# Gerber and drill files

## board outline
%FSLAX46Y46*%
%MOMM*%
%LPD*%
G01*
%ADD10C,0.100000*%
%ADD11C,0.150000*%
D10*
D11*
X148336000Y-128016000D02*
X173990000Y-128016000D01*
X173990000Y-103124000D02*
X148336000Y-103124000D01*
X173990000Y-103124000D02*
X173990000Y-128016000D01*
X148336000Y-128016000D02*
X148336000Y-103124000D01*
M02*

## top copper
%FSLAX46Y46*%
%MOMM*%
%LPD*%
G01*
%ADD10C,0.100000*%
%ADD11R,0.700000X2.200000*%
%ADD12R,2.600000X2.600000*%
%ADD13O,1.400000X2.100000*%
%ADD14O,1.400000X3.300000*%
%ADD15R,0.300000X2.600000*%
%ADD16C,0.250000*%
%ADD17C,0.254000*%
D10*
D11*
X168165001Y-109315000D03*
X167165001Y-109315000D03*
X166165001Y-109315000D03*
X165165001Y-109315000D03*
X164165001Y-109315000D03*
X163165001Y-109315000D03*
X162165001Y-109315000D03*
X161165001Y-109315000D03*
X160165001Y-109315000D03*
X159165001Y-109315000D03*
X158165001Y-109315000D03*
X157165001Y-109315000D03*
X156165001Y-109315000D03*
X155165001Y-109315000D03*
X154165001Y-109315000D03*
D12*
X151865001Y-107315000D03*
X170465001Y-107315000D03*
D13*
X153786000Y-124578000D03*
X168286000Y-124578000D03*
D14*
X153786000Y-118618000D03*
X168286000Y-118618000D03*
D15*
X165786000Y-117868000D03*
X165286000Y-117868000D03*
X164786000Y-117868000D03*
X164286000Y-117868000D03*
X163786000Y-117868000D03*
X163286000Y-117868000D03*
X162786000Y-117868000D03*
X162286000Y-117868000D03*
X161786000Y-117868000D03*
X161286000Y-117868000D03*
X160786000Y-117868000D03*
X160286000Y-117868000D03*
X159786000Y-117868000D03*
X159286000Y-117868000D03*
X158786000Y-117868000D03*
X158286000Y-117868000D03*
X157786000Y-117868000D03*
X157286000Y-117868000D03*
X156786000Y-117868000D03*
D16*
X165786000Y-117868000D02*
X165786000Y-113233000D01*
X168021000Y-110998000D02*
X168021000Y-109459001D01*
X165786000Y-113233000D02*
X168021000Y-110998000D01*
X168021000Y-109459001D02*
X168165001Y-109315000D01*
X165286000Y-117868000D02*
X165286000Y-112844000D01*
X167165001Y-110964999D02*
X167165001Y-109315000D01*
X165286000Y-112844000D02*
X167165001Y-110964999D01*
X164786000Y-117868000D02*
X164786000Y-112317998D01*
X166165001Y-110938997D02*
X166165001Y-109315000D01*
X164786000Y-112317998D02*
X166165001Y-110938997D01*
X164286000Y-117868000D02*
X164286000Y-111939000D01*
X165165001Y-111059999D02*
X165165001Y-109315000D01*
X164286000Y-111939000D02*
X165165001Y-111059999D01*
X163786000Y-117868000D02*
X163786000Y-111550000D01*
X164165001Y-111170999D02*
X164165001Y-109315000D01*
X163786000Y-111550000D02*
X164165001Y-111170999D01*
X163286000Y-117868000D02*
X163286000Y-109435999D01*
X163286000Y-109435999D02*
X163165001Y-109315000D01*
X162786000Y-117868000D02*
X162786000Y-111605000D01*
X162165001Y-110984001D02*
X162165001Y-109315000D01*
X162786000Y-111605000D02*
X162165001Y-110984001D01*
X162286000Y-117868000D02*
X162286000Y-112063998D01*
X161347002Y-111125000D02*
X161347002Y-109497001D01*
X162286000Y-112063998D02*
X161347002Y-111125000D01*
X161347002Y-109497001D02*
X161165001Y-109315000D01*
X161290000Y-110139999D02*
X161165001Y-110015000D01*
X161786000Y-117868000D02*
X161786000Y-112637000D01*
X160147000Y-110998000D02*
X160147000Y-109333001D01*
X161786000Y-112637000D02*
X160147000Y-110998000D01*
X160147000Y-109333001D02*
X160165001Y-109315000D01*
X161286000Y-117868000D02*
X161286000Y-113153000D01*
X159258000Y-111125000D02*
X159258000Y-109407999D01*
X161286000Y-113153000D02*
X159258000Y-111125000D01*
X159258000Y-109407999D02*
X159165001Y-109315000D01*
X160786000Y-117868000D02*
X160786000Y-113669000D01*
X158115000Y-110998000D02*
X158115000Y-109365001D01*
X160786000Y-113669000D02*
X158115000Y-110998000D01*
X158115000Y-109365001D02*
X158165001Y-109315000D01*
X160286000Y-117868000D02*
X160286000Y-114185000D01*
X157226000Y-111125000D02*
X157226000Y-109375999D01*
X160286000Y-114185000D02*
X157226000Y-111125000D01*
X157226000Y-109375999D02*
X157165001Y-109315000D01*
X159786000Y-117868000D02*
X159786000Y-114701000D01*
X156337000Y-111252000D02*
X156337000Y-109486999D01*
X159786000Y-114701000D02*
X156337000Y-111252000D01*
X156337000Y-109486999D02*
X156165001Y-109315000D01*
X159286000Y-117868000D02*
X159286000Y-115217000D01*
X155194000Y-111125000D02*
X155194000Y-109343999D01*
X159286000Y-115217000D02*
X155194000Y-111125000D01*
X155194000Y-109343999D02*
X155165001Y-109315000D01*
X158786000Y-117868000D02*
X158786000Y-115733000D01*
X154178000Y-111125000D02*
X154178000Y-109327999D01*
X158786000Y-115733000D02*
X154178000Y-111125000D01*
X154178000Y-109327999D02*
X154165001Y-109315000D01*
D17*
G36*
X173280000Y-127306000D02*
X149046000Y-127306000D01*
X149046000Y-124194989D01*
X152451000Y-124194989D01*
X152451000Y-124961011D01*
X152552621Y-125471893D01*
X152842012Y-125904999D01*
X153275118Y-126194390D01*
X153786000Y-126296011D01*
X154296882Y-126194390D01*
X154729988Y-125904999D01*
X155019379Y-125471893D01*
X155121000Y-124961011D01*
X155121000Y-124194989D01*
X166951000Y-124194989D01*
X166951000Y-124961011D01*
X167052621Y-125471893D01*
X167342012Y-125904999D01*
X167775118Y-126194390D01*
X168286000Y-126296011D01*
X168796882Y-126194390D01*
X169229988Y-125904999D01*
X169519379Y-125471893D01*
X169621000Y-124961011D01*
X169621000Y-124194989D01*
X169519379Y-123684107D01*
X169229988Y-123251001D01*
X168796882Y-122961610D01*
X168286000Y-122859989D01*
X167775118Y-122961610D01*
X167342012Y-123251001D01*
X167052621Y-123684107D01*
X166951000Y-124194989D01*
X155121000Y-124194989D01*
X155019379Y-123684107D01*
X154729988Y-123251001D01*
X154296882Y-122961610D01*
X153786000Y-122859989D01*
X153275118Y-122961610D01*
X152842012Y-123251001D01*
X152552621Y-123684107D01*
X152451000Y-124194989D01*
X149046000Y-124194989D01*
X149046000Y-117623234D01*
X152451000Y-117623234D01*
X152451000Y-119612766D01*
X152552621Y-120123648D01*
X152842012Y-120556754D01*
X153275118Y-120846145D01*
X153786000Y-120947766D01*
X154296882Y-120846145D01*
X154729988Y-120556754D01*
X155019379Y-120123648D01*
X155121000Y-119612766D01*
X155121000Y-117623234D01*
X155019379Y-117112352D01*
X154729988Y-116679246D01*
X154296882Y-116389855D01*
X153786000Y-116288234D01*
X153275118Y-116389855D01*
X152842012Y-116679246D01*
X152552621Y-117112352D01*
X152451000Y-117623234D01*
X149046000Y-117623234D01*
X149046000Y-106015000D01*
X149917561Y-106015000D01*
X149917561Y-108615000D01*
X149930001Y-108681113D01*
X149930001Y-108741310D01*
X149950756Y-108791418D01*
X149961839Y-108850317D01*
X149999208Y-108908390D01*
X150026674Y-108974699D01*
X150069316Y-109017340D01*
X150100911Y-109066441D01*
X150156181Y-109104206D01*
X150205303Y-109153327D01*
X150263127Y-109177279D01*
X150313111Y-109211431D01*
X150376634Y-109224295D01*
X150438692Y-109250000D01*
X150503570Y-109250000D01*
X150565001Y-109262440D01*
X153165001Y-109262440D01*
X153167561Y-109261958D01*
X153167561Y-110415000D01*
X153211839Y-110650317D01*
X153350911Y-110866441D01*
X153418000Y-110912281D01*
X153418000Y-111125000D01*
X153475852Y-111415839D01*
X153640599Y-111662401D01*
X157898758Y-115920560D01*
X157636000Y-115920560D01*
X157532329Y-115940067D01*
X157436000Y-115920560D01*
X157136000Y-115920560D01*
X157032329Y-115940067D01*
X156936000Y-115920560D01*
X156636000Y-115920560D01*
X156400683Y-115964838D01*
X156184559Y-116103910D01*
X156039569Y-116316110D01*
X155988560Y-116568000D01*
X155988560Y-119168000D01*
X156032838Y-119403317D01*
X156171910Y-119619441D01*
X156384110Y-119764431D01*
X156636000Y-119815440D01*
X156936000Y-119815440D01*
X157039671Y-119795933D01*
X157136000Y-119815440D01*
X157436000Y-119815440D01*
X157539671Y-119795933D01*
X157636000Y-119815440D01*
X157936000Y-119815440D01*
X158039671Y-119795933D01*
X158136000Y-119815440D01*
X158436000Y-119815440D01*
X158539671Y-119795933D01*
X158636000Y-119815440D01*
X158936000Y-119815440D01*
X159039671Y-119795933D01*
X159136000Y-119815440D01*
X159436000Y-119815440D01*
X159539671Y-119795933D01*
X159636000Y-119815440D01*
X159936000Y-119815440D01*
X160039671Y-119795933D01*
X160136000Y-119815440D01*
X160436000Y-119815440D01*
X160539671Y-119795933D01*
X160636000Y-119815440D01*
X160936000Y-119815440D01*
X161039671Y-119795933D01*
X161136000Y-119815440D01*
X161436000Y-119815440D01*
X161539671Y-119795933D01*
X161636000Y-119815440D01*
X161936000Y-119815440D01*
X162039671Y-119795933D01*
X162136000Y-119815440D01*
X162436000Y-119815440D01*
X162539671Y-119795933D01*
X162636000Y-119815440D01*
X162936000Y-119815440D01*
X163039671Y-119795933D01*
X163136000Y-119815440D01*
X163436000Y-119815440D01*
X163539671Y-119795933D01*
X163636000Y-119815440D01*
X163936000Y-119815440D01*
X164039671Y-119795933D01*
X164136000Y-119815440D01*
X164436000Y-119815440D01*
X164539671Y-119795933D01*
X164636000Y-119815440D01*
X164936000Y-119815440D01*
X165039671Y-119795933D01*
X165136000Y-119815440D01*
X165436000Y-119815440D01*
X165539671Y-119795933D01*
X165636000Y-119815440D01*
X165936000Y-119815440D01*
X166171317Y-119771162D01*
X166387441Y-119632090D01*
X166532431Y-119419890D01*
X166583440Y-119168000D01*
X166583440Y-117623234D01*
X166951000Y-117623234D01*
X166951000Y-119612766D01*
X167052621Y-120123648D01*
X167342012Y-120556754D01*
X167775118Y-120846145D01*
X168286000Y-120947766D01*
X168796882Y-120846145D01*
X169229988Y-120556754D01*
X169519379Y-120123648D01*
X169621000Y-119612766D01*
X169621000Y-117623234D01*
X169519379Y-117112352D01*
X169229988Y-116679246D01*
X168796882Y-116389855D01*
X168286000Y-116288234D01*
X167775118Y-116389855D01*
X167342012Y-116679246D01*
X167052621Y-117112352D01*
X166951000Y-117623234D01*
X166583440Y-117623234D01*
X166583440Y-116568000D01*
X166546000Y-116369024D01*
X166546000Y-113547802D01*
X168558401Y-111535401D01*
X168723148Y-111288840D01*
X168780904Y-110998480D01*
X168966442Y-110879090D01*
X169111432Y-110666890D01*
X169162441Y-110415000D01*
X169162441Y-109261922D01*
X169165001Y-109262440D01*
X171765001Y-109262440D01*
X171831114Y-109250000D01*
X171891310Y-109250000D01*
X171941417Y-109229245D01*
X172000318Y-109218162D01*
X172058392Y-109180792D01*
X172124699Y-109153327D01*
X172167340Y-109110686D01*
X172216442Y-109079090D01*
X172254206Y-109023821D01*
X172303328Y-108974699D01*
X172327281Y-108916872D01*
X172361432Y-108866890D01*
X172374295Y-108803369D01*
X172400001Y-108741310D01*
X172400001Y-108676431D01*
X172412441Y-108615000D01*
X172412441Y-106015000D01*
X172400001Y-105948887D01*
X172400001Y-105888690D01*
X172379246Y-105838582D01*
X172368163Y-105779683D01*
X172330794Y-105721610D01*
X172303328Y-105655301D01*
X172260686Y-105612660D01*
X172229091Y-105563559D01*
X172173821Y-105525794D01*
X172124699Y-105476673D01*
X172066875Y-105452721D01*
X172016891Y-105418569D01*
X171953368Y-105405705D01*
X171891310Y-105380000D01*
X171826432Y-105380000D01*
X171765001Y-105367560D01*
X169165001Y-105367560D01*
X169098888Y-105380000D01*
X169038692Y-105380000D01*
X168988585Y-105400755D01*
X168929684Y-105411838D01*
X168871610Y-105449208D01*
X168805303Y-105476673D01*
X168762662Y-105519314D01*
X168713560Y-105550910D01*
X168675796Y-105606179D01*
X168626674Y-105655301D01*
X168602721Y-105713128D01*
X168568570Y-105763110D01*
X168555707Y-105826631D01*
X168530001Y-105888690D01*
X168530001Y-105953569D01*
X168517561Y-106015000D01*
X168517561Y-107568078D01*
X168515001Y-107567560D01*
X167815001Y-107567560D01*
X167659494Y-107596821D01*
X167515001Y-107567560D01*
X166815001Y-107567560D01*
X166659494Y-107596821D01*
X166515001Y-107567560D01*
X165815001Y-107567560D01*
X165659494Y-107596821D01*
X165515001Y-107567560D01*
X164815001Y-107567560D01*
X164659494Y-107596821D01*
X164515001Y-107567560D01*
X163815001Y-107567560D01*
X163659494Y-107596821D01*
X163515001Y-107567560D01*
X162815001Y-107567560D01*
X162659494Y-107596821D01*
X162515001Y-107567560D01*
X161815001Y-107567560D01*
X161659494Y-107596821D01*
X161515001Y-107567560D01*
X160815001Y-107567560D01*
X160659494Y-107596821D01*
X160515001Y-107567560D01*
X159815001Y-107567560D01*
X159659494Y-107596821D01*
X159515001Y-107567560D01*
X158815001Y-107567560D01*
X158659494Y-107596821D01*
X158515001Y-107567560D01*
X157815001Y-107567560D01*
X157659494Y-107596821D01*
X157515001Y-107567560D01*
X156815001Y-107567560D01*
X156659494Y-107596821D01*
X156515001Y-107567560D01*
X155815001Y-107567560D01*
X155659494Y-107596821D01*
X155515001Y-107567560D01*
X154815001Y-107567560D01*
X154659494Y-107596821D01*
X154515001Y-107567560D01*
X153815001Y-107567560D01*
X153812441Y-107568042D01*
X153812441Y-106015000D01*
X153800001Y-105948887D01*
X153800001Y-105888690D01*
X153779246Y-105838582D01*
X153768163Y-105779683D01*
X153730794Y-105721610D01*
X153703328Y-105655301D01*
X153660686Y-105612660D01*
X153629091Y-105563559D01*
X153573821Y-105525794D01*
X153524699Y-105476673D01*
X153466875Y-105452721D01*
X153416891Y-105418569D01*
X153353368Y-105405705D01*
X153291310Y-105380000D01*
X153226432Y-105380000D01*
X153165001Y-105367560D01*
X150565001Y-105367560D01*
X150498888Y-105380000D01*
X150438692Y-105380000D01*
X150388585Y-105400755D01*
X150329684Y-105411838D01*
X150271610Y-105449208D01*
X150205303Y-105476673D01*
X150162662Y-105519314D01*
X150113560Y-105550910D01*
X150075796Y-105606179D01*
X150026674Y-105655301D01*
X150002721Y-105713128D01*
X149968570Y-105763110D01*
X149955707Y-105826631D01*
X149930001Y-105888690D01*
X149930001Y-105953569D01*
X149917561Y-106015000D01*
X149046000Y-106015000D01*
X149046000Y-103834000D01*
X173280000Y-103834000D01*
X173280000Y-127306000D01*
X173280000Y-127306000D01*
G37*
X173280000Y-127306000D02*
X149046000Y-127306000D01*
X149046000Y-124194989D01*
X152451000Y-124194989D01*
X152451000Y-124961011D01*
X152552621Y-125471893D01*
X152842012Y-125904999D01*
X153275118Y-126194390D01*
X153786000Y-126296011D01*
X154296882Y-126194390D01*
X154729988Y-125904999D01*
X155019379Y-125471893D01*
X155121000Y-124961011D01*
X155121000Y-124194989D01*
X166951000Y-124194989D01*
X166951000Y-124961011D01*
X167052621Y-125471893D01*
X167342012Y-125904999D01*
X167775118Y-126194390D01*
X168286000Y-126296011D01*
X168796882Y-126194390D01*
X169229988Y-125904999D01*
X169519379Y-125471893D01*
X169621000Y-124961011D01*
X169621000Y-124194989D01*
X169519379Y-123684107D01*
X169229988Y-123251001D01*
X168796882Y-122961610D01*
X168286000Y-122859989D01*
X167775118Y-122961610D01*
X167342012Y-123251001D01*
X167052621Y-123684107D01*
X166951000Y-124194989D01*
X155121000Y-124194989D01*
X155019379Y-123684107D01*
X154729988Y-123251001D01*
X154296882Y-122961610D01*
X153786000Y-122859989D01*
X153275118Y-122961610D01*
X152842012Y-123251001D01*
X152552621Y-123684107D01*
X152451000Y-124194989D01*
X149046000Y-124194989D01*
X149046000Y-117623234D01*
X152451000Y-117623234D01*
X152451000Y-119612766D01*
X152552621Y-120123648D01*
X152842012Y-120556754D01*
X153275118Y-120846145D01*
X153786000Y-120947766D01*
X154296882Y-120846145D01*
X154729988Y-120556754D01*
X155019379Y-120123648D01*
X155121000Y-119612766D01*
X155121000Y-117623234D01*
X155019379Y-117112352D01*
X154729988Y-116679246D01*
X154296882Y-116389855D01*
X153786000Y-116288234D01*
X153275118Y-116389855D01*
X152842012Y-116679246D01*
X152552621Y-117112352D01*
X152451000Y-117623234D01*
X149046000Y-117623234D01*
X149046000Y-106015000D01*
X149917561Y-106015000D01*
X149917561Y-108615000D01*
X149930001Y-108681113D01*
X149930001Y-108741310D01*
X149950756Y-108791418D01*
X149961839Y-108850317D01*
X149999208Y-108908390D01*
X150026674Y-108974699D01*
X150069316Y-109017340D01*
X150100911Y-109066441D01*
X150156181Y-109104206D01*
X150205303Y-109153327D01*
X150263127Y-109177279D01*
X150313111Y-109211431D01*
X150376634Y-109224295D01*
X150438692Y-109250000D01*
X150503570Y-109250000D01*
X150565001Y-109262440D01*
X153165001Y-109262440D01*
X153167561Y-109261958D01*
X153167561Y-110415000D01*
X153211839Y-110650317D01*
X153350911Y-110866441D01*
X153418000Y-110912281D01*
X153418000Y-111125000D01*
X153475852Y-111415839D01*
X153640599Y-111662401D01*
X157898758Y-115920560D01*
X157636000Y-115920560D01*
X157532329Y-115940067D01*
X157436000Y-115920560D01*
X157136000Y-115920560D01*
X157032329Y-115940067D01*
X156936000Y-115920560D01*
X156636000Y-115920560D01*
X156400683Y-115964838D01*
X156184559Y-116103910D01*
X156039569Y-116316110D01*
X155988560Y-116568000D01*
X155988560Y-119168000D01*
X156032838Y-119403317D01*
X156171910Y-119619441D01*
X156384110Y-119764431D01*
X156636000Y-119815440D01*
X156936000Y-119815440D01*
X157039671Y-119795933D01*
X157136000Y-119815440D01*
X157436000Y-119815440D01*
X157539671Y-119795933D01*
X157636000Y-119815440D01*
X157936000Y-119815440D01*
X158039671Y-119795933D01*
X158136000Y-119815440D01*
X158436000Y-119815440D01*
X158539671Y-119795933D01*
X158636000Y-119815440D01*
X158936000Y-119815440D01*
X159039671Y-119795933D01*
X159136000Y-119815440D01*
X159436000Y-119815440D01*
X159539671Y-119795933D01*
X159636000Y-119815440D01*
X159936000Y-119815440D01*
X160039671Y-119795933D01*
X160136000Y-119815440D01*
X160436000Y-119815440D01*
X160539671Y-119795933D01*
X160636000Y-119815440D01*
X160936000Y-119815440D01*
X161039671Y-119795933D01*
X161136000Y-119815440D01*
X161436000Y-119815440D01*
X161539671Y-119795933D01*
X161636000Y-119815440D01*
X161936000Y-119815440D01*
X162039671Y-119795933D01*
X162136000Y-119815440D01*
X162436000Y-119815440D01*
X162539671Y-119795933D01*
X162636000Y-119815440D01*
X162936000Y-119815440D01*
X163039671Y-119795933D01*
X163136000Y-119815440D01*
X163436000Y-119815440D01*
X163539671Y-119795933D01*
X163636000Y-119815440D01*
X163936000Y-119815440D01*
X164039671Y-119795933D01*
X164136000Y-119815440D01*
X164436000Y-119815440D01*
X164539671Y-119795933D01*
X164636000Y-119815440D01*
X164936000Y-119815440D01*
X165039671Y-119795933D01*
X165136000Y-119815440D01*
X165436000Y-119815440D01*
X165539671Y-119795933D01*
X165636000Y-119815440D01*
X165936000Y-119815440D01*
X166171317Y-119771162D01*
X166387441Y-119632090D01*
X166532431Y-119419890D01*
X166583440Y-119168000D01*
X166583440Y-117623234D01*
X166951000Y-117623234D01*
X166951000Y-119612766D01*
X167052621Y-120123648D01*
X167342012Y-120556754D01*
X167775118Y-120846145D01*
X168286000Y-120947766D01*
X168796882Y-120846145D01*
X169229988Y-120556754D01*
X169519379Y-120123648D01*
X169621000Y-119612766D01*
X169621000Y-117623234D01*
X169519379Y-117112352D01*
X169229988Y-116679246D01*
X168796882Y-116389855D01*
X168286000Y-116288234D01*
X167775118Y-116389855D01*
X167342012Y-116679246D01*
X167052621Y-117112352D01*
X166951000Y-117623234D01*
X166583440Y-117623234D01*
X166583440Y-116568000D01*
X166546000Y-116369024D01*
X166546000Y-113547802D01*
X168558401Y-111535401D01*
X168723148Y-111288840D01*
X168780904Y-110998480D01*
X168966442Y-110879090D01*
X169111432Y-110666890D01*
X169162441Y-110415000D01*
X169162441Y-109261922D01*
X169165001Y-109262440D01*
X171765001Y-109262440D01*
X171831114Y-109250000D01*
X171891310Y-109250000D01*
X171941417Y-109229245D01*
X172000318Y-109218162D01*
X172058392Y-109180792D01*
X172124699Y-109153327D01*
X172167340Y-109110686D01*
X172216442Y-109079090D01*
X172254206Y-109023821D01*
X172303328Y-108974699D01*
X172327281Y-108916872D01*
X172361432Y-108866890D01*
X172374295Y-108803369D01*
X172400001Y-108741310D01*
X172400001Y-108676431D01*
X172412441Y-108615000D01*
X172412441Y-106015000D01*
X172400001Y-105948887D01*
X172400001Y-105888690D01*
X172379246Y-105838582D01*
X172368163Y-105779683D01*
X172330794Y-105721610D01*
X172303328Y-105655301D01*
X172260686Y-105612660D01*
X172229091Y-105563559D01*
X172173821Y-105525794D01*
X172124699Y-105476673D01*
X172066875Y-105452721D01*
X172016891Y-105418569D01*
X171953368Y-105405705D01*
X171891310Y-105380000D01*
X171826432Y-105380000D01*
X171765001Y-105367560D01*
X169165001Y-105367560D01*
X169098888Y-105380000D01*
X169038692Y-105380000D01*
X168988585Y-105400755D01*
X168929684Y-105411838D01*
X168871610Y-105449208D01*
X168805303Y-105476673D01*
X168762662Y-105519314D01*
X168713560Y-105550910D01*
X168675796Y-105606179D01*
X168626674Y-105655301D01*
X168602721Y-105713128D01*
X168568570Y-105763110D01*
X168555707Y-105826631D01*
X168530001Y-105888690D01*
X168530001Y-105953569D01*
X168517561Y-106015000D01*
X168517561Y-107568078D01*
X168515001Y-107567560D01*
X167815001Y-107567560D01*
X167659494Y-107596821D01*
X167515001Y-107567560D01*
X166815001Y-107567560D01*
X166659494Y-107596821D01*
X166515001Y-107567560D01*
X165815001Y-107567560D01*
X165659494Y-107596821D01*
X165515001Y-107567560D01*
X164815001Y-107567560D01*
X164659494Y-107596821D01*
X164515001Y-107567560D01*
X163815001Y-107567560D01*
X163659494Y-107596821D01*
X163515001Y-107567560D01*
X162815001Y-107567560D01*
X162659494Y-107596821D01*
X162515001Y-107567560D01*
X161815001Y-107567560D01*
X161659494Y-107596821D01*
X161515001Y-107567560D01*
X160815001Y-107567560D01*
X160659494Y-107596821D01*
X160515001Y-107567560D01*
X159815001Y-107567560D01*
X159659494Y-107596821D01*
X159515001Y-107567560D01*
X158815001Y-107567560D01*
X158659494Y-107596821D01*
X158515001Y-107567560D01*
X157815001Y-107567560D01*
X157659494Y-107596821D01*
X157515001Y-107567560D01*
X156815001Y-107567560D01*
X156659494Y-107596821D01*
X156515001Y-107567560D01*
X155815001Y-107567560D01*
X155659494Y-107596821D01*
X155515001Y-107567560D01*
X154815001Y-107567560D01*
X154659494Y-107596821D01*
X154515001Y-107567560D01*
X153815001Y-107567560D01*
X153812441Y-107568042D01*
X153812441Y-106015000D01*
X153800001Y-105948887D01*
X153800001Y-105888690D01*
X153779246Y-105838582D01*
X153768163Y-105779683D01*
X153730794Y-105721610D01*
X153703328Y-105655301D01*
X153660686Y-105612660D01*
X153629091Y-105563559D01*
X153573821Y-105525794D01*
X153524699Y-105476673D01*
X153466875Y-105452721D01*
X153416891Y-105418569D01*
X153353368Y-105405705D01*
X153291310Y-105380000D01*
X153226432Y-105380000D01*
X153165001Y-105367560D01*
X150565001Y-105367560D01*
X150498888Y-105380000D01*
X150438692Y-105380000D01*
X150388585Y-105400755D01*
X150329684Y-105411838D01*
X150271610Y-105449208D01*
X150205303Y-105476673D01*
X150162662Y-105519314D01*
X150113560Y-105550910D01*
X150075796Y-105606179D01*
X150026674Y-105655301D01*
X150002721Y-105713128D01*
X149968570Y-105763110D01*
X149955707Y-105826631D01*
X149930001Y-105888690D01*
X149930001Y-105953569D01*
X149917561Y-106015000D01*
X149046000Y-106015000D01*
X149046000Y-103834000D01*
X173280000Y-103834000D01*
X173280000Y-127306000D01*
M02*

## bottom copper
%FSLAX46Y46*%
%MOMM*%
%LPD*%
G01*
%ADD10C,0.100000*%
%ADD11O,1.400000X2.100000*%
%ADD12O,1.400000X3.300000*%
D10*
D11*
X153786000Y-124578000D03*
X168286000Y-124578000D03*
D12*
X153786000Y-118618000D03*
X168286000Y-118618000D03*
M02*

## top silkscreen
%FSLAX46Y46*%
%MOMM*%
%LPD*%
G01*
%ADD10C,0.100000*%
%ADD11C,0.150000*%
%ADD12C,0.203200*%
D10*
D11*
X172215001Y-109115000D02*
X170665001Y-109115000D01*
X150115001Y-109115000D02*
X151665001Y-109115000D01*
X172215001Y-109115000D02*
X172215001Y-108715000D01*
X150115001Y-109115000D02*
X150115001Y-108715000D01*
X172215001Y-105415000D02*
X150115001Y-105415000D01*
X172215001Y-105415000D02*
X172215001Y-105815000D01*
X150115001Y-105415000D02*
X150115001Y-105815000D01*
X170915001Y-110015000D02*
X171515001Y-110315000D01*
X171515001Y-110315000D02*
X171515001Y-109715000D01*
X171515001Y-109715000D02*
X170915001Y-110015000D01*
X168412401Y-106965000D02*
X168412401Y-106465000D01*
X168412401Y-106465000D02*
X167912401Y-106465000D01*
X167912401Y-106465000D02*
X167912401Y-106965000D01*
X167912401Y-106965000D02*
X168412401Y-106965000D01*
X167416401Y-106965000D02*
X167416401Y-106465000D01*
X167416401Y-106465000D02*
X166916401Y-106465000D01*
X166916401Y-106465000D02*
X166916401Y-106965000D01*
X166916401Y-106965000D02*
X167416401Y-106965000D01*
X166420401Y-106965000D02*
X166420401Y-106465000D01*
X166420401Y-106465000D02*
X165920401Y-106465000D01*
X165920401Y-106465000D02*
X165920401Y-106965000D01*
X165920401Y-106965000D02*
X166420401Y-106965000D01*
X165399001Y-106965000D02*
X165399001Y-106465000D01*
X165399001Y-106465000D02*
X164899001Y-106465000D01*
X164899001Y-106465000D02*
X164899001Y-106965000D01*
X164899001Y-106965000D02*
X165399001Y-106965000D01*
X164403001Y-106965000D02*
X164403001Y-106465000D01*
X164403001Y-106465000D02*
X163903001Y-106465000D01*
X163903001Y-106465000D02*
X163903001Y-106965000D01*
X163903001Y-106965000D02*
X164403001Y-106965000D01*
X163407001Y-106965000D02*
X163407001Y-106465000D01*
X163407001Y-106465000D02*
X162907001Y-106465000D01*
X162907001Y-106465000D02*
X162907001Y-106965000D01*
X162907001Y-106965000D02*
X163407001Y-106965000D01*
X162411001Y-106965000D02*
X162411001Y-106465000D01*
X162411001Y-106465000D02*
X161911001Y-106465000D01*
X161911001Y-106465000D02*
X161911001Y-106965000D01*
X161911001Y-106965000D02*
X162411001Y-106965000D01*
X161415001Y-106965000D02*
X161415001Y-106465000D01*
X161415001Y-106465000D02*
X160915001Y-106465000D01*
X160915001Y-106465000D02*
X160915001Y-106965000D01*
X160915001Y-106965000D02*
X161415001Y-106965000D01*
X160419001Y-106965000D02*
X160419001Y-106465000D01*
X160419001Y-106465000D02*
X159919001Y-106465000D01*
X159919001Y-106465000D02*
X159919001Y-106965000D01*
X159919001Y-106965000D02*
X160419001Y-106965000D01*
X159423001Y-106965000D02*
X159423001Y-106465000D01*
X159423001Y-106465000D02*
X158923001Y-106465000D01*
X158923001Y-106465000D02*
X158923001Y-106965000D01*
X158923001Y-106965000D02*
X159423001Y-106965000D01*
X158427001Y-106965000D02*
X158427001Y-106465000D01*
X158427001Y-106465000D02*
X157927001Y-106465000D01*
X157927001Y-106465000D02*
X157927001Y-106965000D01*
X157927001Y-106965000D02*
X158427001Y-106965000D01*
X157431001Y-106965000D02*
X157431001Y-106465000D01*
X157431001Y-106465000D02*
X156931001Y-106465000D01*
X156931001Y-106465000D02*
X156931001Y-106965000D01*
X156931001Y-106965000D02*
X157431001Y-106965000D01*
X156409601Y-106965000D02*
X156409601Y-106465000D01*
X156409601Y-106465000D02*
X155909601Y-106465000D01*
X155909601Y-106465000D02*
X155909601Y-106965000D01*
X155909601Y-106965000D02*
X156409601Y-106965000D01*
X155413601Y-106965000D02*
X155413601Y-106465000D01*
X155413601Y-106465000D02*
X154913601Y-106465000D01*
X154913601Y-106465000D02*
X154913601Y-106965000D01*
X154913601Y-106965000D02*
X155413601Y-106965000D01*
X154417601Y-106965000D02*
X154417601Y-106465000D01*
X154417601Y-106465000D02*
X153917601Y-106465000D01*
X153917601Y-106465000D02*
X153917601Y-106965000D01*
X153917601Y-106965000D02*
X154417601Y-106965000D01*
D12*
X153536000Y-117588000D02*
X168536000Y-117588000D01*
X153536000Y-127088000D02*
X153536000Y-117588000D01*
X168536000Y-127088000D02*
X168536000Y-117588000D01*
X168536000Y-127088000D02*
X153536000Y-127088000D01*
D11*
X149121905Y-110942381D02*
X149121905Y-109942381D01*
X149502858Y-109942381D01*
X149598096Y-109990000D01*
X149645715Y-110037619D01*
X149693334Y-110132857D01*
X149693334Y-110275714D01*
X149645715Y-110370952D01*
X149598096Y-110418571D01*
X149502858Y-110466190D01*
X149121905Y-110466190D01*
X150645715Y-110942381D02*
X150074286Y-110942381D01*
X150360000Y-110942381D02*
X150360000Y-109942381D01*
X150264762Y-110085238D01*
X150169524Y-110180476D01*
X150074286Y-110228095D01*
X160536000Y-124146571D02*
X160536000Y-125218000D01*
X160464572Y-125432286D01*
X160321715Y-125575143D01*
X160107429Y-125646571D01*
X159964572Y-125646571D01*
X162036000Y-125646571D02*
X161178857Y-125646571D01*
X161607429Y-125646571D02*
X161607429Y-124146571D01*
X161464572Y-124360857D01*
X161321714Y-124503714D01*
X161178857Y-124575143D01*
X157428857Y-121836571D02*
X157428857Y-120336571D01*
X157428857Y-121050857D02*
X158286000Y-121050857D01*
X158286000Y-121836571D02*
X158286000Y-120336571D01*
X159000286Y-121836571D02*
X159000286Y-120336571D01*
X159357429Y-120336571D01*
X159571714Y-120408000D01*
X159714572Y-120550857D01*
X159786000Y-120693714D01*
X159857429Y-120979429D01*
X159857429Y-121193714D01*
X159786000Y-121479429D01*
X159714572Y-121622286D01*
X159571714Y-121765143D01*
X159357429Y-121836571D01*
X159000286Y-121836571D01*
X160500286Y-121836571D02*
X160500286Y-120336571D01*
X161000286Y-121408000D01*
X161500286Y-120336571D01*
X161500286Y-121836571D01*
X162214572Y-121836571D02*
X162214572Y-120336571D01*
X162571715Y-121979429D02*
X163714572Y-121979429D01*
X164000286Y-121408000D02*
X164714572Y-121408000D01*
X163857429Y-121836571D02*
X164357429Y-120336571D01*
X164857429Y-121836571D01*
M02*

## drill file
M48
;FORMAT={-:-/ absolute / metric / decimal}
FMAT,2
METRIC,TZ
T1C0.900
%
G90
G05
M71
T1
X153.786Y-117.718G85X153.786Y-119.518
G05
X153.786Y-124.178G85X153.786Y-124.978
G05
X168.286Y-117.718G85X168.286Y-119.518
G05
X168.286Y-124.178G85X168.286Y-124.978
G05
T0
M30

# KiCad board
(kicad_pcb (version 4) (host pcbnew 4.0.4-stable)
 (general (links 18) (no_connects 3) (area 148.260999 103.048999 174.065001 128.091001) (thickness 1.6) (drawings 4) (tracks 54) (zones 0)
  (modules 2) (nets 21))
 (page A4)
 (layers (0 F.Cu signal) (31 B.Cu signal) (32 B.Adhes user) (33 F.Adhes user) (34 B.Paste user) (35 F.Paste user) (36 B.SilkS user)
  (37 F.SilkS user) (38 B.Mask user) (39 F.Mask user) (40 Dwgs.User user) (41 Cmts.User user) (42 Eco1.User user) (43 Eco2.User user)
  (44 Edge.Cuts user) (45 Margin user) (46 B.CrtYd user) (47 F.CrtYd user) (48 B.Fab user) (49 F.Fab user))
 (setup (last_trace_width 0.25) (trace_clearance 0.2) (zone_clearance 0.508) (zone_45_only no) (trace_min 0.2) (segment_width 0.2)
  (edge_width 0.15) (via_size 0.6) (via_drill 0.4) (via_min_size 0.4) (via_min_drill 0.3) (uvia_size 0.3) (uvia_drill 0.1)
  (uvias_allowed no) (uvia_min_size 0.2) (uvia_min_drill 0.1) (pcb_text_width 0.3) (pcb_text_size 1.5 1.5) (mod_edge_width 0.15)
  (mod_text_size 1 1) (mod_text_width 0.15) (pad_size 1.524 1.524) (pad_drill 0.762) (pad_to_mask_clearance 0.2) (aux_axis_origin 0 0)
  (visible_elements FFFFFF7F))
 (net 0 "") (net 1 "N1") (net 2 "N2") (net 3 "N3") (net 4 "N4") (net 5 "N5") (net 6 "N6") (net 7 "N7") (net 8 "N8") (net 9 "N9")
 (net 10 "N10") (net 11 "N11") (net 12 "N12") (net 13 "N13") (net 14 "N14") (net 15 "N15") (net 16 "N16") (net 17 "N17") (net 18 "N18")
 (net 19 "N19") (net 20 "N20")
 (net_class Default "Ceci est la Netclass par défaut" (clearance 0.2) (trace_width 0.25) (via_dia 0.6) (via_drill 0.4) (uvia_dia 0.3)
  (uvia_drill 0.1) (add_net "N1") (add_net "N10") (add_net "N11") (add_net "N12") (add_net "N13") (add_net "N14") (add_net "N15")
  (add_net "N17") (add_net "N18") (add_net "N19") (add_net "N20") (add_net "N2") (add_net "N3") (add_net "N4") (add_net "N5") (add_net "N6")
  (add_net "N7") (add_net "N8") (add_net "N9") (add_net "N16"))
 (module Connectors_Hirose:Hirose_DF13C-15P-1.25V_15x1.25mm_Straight (layer F.Cu) (at 161.165001 108.615 180)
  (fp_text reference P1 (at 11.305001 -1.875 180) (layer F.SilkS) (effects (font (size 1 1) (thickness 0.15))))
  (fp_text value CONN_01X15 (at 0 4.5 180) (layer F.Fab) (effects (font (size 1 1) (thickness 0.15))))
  (fp_line (start -11.05 -0.5) (end -9.5 -0.5) (layer F.SilkS) (width 0.15))
  (fp_line (start 11.05 -0.5) (end 9.5 -0.5) (layer F.SilkS) (width 0.15))
  (fp_line (start -11.05 -0.5) (end -11.05 -0.1) (layer F.SilkS) (width 0.15))
  (fp_line (start 11.05 -0.5) (end 11.05 -0.1) (layer F.SilkS) (width 0.15))
  (fp_line (start -11.05 3.2) (end 11.05 3.2) (layer F.SilkS) (width 0.15))
  (fp_line (start -11.05 3.2) (end -11.05 2.8) (layer F.SilkS) (width 0.15))
  (fp_line (start 11.05 3.2) (end 11.05 2.8) (layer F.SilkS) (width 0.15))
  (fp_line (start -9.75 -1.4) (end -10.35 -1.7) (layer F.SilkS) (width 0.15))
  (fp_line (start -10.35 -1.7) (end -10.35 -1.1) (layer F.SilkS) (width 0.15))
  (fp_line (start -10.35 -1.1) (end -9.75 -1.4) (layer F.SilkS) (width 0.15))
  (fp_line (start -7.2474 1.65) (end -7.2474 2.15) (layer F.SilkS) (width 0.15))
  (fp_line (start -7.2474 2.15) (end -6.7474 2.15) (layer F.SilkS) (width 0.15))
  (fp_line (start -6.7474 2.15) (end -6.7474 1.65) (layer F.SilkS) (width 0.15))
  (fp_line (start -6.7474 1.65) (end -7.2474 1.65) (layer F.SilkS) (width 0.15))
  (fp_line (start -6.2514 1.65) (end -6.2514 2.15) (layer F.SilkS) (width 0.15))
  (fp_line (start -6.2514 2.15) (end -5.7514 2.15) (layer F.SilkS) (width 0.15))
  (fp_line (start -5.7514 2.15) (end -5.7514 1.65) (layer F.SilkS) (width 0.15))
  (fp_line (start -5.7514 1.65) (end -6.2514 1.65) (layer F.SilkS) (width 0.15))
  (fp_line (start -5.2554 1.65) (end -5.2554 2.15) (layer F.SilkS) (width 0.15))
  (fp_line (start -5.2554 2.15) (end -4.7554 2.15) (layer F.SilkS) (width 0.15))
  (fp_line (start -4.7554 2.15) (end -4.7554 1.65) (layer F.SilkS) (width 0.15))
  (fp_line (start -4.7554 1.65) (end -5.2554 1.65) (layer F.SilkS) (width 0.15))
  (fp_line (start -4.234 1.65) (end -4.234 2.15) (layer F.SilkS) (width 0.15))
  (fp_line (start -4.234 2.15) (end -3.734 2.15) (layer F.SilkS) (width 0.15))
  (fp_line (start -3.734 2.15) (end -3.734 1.65) (layer F.SilkS) (width 0.15))
  (fp_line (start -3.734 1.65) (end -4.234 1.65) (layer F.SilkS) (width 0.15))
  (fp_line (start -3.238 1.65) (end -3.238 2.15) (layer F.SilkS) (width 0.15))
  (fp_line (start -3.238 2.15) (end -2.738 2.15) (layer F.SilkS) (width 0.15))
  (fp_line (start -2.738 2.15) (end -2.738 1.65) (layer F.SilkS) (width 0.15))
  (fp_line (start -2.738 1.65) (end -3.238 1.65) (layer F.SilkS) (width 0.15))
  (fp_line (start -2.242 1.65) (end -2.242 2.15) (layer F.SilkS) (width 0.15))
  (fp_line (start -2.242 2.15) (end -1.742 2.15) (layer F.SilkS) (width 0.15))
  (fp_line (start -1.742 2.15) (end -1.742 1.65) (layer F.SilkS) (width 0.15))
  (fp_line (start -1.742 1.65) (end -2.242 1.65) (layer F.SilkS) (width 0.15))
  (fp_line (start -1.246 1.65) (end -1.246 2.15) (layer F.SilkS) (width 0.15))
  (fp_line (start -1.246 2.15) (end -0.746 2.15) (layer F.SilkS) (width 0.15))
  (fp_line (start -0.746 2.15) (end -0.746 1.65) (layer F.SilkS) (width 0.15))
  (fp_line (start -0.746 1.65) (end -1.246 1.65) (layer F.SilkS) (width 0.15))
  (fp_line (start -0.25 1.65) (end -0.25 2.15) (layer F.SilkS) (width 0.15))
  (fp_line (start -0.25 2.15) (end 0.25 2.15) (layer F.SilkS) (width 0.15))
  (fp_line (start 0.25 2.15) (end 0.25 1.65) (layer F.SilkS) (width 0.15))
  (fp_line (start 0.25 1.65) (end -0.25 1.65) (layer F.SilkS) (width 0.15))
  (fp_line (start 0.746 1.65) (end 0.746 2.15) (layer F.SilkS) (width 0.15))
  (fp_line (start 0.746 2.15) (end 1.246 2.15) (layer F.SilkS) (width 0.15))
  (fp_line (start 1.246 2.15) (end 1.246 1.65) (layer F.SilkS) (width 0.15))
  (fp_line (start 1.246 1.65) (end 0.746 1.65) (layer F.SilkS) (width 0.15))
  (fp_line (start 1.742 1.65) (end 1.742 2.15) (layer F.SilkS) (width 0.15))
  (fp_line (start 1.742 2.15) (end 2.242 2.15) (layer F.SilkS) (width 0.15))
  (fp_line (start 2.242 2.15) (end 2.242 1.65) (layer F.SilkS) (width 0.15))
  (fp_line (start 2.242 1.65) (end 1.742 1.65) (layer F.SilkS) (width 0.15))
  (fp_line (start 2.738 1.65) (end 2.738 2.15) (layer F.SilkS) (width 0.15))
  (fp_line (start 2.738 2.15) (end 3.238 2.15) (layer F.SilkS) (width 0.15))
  (fp_line (start 3.238 2.15) (end 3.238 1.65) (layer F.SilkS) (width 0.15))
  (fp_line (start 3.238 1.65) (end 2.738 1.65) (layer F.SilkS) (width 0.15))
  (fp_line (start 3.734 1.65) (end 3.734 2.15) (layer F.SilkS) (width 0.15))
  (fp_line (start 3.734 2.15) (end 4.234 2.15) (layer F.SilkS) (width 0.15))
  (fp_line (start 4.234 2.15) (end 4.234 1.65) (layer F.SilkS) (width 0.15))
  (fp_line (start 4.234 1.65) (end 3.734 1.65) (layer F.SilkS) (width 0.15))
  (fp_line (start 4.7554 1.65) (end 4.7554 2.15) (layer F.SilkS) (width 0.15))
  (fp_line (start 4.7554 2.15) (end 5.2554 2.15) (layer F.SilkS) (width 0.15))
  (fp_line (start 5.2554 2.15) (end 5.2554 1.65) (layer F.SilkS) (width 0.15))
  (fp_line (start 5.2554 1.65) (end 4.7554 1.65) (layer F.SilkS) (width 0.15))
  (fp_line (start 5.7514 1.65) (end 5.7514 2.15) (layer F.SilkS) (width 0.15))
  (fp_line (start 5.7514 2.15) (end 6.2514 2.15) (layer F.SilkS) (width 0.15))
  (fp_line (start 6.2514 2.15) (end 6.2514 1.65) (layer F.SilkS) (width 0.15))
  (fp_line (start 6.2514 1.65) (end 5.7514 1.65) (layer F.SilkS) (width 0.15))
  (fp_line (start 6.7474 1.65) (end 6.7474 2.15) (layer F.SilkS) (width 0.15))
  (fp_line (start 6.7474 2.15) (end 7.2474 2.15) (layer F.SilkS) (width 0.15))
  (fp_line (start 7.2474 2.15) (end 7.2474 1.65) (layer F.SilkS) (width 0.15))
  (fp_line (start 7.2474 1.65) (end 6.7474 1.65) (layer F.SilkS) (width 0.15))
  (pad 1 smd rect (at -7 -0.7 180) (size 0.7 2.2) (layers F.Cu F.Paste F.Mask) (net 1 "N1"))
  (pad 2 smd rect (at -6 -0.7 180) (size 0.7 2.2) (layers F.Cu F.Paste F.Mask) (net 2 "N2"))
  (pad 3 smd rect (at -5 -0.7 180) (size 0.7 2.2) (layers F.Cu F.Paste F.Mask) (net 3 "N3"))
  (pad 4 smd rect (at -4 -0.7 180) (size 0.7 2.2) (layers F.Cu F.Paste F.Mask) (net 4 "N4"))
  (pad 5 smd rect (at -3 -0.7 180) (size 0.7 2.2) (layers F.Cu F.Paste F.Mask) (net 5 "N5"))
  (pad 6 smd rect (at -2 -0.7 180) (size 0.7 2.2) (layers F.Cu F.Paste F.Mask) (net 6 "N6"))
  (pad 7 smd rect (at -1 -0.7 180) (size 0.7 2.2) (layers F.Cu F.Paste F.Mask) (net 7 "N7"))
  (pad 8 smd rect (at 0 -0.7 180) (size 0.7 2.2) (layers F.Cu F.Paste F.Mask) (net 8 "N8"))
  (pad 9 smd rect (at 1 -0.7 180) (size 0.7 2.2) (layers F.Cu F.Paste F.Mask) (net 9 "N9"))
  (pad 10 smd rect (at 2 -0.7 180) (size 0.7 2.2) (layers F.Cu F.Paste F.Mask) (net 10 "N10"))
  (pad 11 smd rect (at 3 -0.7 180) (size 0.7 2.2) (layers F.Cu F.Paste F.Mask) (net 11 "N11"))
  (pad 12 smd rect (at 4 -0.7 180) (size 0.7 2.2) (layers F.Cu F.Paste F.Mask) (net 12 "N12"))
  (pad 13 smd rect (at 5 -0.7 180) (size 0.7 2.2) (layers F.Cu F.Paste F.Mask) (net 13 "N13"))
  (pad 14 smd rect (at 6 -0.7 180) (size 0.7 2.2) (layers F.Cu F.Paste F.Mask) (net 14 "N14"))
  (pad 15 smd rect (at 7 -0.7 180) (size 0.7 2.2) (layers F.Cu F.Paste F.Mask) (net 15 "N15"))
  (pad "" smd rect (at 9.3 1.3 180) (size 2.6 2.6) (layers F.Cu F.Paste F.Mask))
  (pad "" smd rect (at -9.3 1.3 180) (size 2.6 2.6) (layers F.Cu F.Paste F.Mask)))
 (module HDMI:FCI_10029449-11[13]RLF (layer F.Cu) (at 161.036 118.618)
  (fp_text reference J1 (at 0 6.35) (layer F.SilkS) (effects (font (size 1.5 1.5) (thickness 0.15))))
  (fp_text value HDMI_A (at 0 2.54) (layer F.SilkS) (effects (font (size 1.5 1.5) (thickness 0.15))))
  (fp_line (start -7.5 -1.03) (end 7.5 -1.03) (layer F.SilkS) (width 0.2032))
  (fp_line (start -7.5 8.47) (end -7.5 -1.03) (layer F.SilkS) (width 0.2032))
  (fp_line (start 7.5 8.47) (end 7.5 -1.03) (layer F.SilkS) (width 0.2032))
  (fp_line (start 7.5 8.47) (end -7.5 8.47) (layer F.SilkS) (width 0.2032))
  (pad SHLD thru_hole oval (at -7.25 5.96) (size 1.4 2.1) (drill oval 0.9 1.7) (layers *.Cu *.SilkS *.Mask) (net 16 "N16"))
  (pad SHLD thru_hole oval (at 7.25 5.96) (size 1.4 2.1) (drill oval 0.9 1.7) (layers *.Cu *.SilkS *.Mask) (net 16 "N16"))
  (pad SHLD thru_hole oval (at -7.25 0) (size 1.4 3.3) (drill oval 0.9 2.7) (layers *.Cu *.SilkS *.Mask) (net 16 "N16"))
  (pad SHLD thru_hole oval (at 7.25 0) (size 1.4 3.3) (drill oval 0.9 2.7) (layers *.Cu *.SilkS *.Mask) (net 16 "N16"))
  (pad 1 smd rect (at 4.75 -0.75) (size 0.3 2.6) (layers F.Cu F.Paste F.Mask) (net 1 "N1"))
  (pad 2 smd rect (at 4.25 -0.75) (size 0.3 2.6) (layers F.Cu F.Paste F.Mask) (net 2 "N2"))
  (pad 3 smd rect (at 3.75 -0.75) (size 0.3 2.6) (layers F.Cu F.Paste F.Mask) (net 3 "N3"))
  (pad 4 smd rect (at 3.25 -0.75) (size 0.3 2.6) (layers F.Cu F.Paste F.Mask) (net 4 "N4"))
  (pad 5 smd rect (at 2.75 -0.75) (size 0.3 2.6) (layers F.Cu F.Paste F.Mask) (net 5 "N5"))
  (pad 6 smd rect (at 2.25 -0.75) (size 0.3 2.6) (layers F.Cu F.Paste F.Mask) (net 6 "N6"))
  (pad 7 smd rect (at 1.75 -0.75) (size 0.3 2.6) (layers F.Cu F.Paste F.Mask) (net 7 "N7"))
  (pad 8 smd rect (at 1.25 -0.75) (size 0.3 2.6) (layers F.Cu F.Paste F.Mask) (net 8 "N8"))
  (pad 9 smd rect (at 0.75 -0.75) (size 0.3 2.6) (layers F.Cu F.Paste F.Mask) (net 9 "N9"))
  (pad 10 smd rect (at 0.25 -0.75) (size 0.3 2.6) (layers F.Cu F.Paste F.Mask) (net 10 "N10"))
  (pad 11 smd rect (at -0.25 -0.75) (size 0.3 2.6) (layers F.Cu F.Paste F.Mask) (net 11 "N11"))
  (pad 12 smd rect (at -0.75 -0.75) (size 0.3 2.6) (layers F.Cu F.Paste F.Mask) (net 12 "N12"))
  (pad 13 smd rect (at -1.25 -0.75) (size 0.3 2.6) (layers F.Cu F.Paste F.Mask) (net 13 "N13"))
  (pad 14 smd rect (at -1.75 -0.75) (size 0.3 2.6) (layers F.Cu F.Paste F.Mask) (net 14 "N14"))
  (pad 15 smd rect (at -2.25 -0.75) (size 0.3 2.6) (layers F.Cu F.Paste F.Mask) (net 15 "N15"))
  (pad 16 smd rect (at -2.75 -0.75) (size 0.3 2.6) (layers F.Cu F.Paste F.Mask) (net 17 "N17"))
  (pad 17 smd rect (at -3.25 -0.75) (size 0.3 2.6) (layers F.Cu F.Paste F.Mask) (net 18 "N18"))
  (pad 18 smd rect (at -3.75 -0.75) (size 0.3 2.6) (layers F.Cu F.Paste F.Mask) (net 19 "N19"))
  (pad 19 smd rect (at -4.25 -0.75) (size 0.3 2.6) (layers F.Cu F.Paste F.Mask) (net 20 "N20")))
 (gr_line (start 148.336 128.016) (end 173.99 128.016) (angle 90) (layer Edge.Cuts) (width 0.15))
 (gr_line (start 173.99 103.124) (end 148.336 103.124) (angle 90) (layer Edge.Cuts) (width 0.15))
 (gr_line (start 173.99 103.124) (end 173.99 128.016) (angle 90) (layer Edge.Cuts) (width 0.15))
 (gr_line (start 148.336 128.016) (end 148.336 103.124) (angle 90) (layer Edge.Cuts) (width 0.15))
 (segment (start 165.786 117.868) (end 165.786 113.233) (width 0.25) (layer F.Cu) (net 1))
 (segment (start 168.021 110.998) (end 168.021 109.459001) (width 0.25) (layer F.Cu) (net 1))
 (segment (start 165.786 113.233) (end 168.021 110.998) (width 0.25) (layer F.Cu) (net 1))
 (segment (start 168.021 109.459001) (end 168.165001 109.315) (width 0.25) (layer F.Cu) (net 1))
 (segment (start 165.286 117.868) (end 165.286 112.844) (width 0.25) (layer F.Cu) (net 2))
 (segment (start 167.165001 110.964999) (end 167.165001 109.315) (width 0.25) (layer F.Cu) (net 2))
 (segment (start 165.286 112.844) (end 167.165001 110.964999) (width 0.25) (layer F.Cu) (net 2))
 (segment (start 164.786 117.868) (end 164.786 112.317998) (width 0.25) (layer F.Cu) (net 3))
 (segment (start 166.165001 110.938997) (end 166.165001 109.315) (width 0.25) (layer F.Cu) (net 3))
 (segment (start 164.786 112.317998) (end 166.165001 110.938997) (width 0.25) (layer F.Cu) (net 3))
 (segment (start 164.286 117.868) (end 164.286 111.939) (width 0.25) (layer F.Cu) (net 4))
 (segment (start 165.165001 111.059999) (end 165.165001 109.315) (width 0.25) (layer F.Cu) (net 4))
 (segment (start 164.286 111.939) (end 165.165001 111.059999) (width 0.25) (layer F.Cu) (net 4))
 (segment (start 163.786 117.868) (end 163.786 111.55) (width 0.25) (layer F.Cu) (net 5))
 (segment (start 164.165001 111.170999) (end 164.165001 109.315) (width 0.25) (layer F.Cu) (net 5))
 (segment (start 163.786 111.55) (end 164.165001 111.170999) (width 0.25) (layer F.Cu) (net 5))
 (segment (start 163.286 117.868) (end 163.286 109.435999) (width 0.25) (layer F.Cu) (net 6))
 (segment (start 163.286 109.435999) (end 163.165001 109.315) (width 0.25) (layer F.Cu) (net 6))
 (segment (start 162.786 117.868) (end 162.786 111.605) (width 0.25) (layer F.Cu) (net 7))
 (segment (start 162.165001 110.984001) (end 162.165001 109.315) (width 0.25) (layer F.Cu) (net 7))
 (segment (start 162.786 111.605) (end 162.165001 110.984001) (width 0.25) (layer F.Cu) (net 7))
 (segment (start 162.286 117.868) (end 162.286 112.063998) (width 0.25) (layer F.Cu) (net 8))
 (segment (start 161.347002 111.125) (end 161.347002 109.497001) (width 0.25) (layer F.Cu) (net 8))
 (segment (start 162.286 112.063998) (end 161.347002 111.125) (width 0.25) (layer F.Cu) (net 8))
 (segment (start 161.347002 109.497001) (end 161.165001 109.315) (width 0.25) (layer F.Cu) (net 8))
 (segment (start 161.29 110.139999) (end 161.165001 110.015) (width 0.25) (layer F.Cu) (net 8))
 (segment (start 161.786 117.868) (end 161.786 112.637) (width 0.25) (layer F.Cu) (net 9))
 (segment (start 160.147 110.998) (end 160.147 109.333001) (width 0.25) (layer F.Cu) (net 9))
 (segment (start 161.786 112.637) (end 160.147 110.998) (width 0.25) (layer F.Cu) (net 9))
 (segment (start 160.147 109.333001) (end 160.165001 109.315) (width 0.25) (layer F.Cu) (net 9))
 (segment (start 161.286 117.868) (end 161.286 113.153) (width 0.25) (layer F.Cu) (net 10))
 (segment (start 159.258 111.125) (end 159.258 109.407999) (width 0.25) (layer F.Cu) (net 10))
 (segment (start 161.286 113.153) (end 159.258 111.125) (width 0.25) (layer F.Cu) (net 10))
 (segment (start 159.258 109.407999) (end 159.165001 109.315) (width 0.25) (layer F.Cu) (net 10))
 (segment (start 160.786 117.868) (end 160.786 113.669) (width 0.25) (layer F.Cu) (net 11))
 (segment (start 158.115 110.998) (end 158.115 109.365001) (width 0.25) (layer F.Cu) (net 11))
 (segment (start 160.786 113.669) (end 158.115 110.998) (width 0.25) (layer F.Cu) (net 11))
 (segment (start 158.115 109.365001) (end 158.165001 109.315) (width 0.25) (layer F.Cu) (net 11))
 (segment (start 160.286 117.868) (end 160.286 114.185) (width 0.25) (layer F.Cu) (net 12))
 (segment (start 157.226 111.125) (end 157.226 109.375999) (width 0.25) (layer F.Cu) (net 12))
 (segment (start 160.286 114.185) (end 157.226 111.125) (width 0.25) (layer F.Cu) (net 12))
 (segment (start 157.226 109.375999) (end 157.165001 109.315) (width 0.25) (layer F.Cu) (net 12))
 (segment (start 159.786 117.868) (end 159.786 114.701) (width 0.25) (layer F.Cu) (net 13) (status 400000))
 (segment (start 156.337 111.252) (end 156.337 109.486999) (width 0.25) (layer F.Cu) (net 13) (status 800000))
 (segment (start 159.786 114.701) (end 156.337 111.252) (width 0.25) (layer F.Cu) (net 13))
 (segment (start 156.337 109.486999) (end 156.165001 109.315) (width 0.25) (layer F.Cu) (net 13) (status C00000))
 (segment (start 159.286 117.868) (end 159.286 115.217) (width 0.25) (layer F.Cu) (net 14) (status 400000))
 (segment (start 155.194 111.125) (end 155.194 109.343999) (width 0.25) (layer F.Cu) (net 14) (status 800000))
 (segment (start 159.286 115.217) (end 155.194 111.125) (width 0.25) (layer F.Cu) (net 14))
 (segment (start 155.194 109.343999) (end 155.165001 109.315) (width 0.25) (layer F.Cu) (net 14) (status C00000))
 (segment (start 158.786 117.868) (end 158.786 115.733) (width 0.25) (layer F.Cu) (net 15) (status 400000))
 (segment (start 154.178 111.125) (end 154.178 109.327999) (width 0.25) (layer F.Cu) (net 15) (status 800000))
 (segment (start 158.786 115.733) (end 154.178 111.125) (width 0.25) (layer F.Cu) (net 15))
 (segment (start 154.178 109.327999) (end 154.165001 109.315) (width 0.25) (layer F.Cu) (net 15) (status C00000))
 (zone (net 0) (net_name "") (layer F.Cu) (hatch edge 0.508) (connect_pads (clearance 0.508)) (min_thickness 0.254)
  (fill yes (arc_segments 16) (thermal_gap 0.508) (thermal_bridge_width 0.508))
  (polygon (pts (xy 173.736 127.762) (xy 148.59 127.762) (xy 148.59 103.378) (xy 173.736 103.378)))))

